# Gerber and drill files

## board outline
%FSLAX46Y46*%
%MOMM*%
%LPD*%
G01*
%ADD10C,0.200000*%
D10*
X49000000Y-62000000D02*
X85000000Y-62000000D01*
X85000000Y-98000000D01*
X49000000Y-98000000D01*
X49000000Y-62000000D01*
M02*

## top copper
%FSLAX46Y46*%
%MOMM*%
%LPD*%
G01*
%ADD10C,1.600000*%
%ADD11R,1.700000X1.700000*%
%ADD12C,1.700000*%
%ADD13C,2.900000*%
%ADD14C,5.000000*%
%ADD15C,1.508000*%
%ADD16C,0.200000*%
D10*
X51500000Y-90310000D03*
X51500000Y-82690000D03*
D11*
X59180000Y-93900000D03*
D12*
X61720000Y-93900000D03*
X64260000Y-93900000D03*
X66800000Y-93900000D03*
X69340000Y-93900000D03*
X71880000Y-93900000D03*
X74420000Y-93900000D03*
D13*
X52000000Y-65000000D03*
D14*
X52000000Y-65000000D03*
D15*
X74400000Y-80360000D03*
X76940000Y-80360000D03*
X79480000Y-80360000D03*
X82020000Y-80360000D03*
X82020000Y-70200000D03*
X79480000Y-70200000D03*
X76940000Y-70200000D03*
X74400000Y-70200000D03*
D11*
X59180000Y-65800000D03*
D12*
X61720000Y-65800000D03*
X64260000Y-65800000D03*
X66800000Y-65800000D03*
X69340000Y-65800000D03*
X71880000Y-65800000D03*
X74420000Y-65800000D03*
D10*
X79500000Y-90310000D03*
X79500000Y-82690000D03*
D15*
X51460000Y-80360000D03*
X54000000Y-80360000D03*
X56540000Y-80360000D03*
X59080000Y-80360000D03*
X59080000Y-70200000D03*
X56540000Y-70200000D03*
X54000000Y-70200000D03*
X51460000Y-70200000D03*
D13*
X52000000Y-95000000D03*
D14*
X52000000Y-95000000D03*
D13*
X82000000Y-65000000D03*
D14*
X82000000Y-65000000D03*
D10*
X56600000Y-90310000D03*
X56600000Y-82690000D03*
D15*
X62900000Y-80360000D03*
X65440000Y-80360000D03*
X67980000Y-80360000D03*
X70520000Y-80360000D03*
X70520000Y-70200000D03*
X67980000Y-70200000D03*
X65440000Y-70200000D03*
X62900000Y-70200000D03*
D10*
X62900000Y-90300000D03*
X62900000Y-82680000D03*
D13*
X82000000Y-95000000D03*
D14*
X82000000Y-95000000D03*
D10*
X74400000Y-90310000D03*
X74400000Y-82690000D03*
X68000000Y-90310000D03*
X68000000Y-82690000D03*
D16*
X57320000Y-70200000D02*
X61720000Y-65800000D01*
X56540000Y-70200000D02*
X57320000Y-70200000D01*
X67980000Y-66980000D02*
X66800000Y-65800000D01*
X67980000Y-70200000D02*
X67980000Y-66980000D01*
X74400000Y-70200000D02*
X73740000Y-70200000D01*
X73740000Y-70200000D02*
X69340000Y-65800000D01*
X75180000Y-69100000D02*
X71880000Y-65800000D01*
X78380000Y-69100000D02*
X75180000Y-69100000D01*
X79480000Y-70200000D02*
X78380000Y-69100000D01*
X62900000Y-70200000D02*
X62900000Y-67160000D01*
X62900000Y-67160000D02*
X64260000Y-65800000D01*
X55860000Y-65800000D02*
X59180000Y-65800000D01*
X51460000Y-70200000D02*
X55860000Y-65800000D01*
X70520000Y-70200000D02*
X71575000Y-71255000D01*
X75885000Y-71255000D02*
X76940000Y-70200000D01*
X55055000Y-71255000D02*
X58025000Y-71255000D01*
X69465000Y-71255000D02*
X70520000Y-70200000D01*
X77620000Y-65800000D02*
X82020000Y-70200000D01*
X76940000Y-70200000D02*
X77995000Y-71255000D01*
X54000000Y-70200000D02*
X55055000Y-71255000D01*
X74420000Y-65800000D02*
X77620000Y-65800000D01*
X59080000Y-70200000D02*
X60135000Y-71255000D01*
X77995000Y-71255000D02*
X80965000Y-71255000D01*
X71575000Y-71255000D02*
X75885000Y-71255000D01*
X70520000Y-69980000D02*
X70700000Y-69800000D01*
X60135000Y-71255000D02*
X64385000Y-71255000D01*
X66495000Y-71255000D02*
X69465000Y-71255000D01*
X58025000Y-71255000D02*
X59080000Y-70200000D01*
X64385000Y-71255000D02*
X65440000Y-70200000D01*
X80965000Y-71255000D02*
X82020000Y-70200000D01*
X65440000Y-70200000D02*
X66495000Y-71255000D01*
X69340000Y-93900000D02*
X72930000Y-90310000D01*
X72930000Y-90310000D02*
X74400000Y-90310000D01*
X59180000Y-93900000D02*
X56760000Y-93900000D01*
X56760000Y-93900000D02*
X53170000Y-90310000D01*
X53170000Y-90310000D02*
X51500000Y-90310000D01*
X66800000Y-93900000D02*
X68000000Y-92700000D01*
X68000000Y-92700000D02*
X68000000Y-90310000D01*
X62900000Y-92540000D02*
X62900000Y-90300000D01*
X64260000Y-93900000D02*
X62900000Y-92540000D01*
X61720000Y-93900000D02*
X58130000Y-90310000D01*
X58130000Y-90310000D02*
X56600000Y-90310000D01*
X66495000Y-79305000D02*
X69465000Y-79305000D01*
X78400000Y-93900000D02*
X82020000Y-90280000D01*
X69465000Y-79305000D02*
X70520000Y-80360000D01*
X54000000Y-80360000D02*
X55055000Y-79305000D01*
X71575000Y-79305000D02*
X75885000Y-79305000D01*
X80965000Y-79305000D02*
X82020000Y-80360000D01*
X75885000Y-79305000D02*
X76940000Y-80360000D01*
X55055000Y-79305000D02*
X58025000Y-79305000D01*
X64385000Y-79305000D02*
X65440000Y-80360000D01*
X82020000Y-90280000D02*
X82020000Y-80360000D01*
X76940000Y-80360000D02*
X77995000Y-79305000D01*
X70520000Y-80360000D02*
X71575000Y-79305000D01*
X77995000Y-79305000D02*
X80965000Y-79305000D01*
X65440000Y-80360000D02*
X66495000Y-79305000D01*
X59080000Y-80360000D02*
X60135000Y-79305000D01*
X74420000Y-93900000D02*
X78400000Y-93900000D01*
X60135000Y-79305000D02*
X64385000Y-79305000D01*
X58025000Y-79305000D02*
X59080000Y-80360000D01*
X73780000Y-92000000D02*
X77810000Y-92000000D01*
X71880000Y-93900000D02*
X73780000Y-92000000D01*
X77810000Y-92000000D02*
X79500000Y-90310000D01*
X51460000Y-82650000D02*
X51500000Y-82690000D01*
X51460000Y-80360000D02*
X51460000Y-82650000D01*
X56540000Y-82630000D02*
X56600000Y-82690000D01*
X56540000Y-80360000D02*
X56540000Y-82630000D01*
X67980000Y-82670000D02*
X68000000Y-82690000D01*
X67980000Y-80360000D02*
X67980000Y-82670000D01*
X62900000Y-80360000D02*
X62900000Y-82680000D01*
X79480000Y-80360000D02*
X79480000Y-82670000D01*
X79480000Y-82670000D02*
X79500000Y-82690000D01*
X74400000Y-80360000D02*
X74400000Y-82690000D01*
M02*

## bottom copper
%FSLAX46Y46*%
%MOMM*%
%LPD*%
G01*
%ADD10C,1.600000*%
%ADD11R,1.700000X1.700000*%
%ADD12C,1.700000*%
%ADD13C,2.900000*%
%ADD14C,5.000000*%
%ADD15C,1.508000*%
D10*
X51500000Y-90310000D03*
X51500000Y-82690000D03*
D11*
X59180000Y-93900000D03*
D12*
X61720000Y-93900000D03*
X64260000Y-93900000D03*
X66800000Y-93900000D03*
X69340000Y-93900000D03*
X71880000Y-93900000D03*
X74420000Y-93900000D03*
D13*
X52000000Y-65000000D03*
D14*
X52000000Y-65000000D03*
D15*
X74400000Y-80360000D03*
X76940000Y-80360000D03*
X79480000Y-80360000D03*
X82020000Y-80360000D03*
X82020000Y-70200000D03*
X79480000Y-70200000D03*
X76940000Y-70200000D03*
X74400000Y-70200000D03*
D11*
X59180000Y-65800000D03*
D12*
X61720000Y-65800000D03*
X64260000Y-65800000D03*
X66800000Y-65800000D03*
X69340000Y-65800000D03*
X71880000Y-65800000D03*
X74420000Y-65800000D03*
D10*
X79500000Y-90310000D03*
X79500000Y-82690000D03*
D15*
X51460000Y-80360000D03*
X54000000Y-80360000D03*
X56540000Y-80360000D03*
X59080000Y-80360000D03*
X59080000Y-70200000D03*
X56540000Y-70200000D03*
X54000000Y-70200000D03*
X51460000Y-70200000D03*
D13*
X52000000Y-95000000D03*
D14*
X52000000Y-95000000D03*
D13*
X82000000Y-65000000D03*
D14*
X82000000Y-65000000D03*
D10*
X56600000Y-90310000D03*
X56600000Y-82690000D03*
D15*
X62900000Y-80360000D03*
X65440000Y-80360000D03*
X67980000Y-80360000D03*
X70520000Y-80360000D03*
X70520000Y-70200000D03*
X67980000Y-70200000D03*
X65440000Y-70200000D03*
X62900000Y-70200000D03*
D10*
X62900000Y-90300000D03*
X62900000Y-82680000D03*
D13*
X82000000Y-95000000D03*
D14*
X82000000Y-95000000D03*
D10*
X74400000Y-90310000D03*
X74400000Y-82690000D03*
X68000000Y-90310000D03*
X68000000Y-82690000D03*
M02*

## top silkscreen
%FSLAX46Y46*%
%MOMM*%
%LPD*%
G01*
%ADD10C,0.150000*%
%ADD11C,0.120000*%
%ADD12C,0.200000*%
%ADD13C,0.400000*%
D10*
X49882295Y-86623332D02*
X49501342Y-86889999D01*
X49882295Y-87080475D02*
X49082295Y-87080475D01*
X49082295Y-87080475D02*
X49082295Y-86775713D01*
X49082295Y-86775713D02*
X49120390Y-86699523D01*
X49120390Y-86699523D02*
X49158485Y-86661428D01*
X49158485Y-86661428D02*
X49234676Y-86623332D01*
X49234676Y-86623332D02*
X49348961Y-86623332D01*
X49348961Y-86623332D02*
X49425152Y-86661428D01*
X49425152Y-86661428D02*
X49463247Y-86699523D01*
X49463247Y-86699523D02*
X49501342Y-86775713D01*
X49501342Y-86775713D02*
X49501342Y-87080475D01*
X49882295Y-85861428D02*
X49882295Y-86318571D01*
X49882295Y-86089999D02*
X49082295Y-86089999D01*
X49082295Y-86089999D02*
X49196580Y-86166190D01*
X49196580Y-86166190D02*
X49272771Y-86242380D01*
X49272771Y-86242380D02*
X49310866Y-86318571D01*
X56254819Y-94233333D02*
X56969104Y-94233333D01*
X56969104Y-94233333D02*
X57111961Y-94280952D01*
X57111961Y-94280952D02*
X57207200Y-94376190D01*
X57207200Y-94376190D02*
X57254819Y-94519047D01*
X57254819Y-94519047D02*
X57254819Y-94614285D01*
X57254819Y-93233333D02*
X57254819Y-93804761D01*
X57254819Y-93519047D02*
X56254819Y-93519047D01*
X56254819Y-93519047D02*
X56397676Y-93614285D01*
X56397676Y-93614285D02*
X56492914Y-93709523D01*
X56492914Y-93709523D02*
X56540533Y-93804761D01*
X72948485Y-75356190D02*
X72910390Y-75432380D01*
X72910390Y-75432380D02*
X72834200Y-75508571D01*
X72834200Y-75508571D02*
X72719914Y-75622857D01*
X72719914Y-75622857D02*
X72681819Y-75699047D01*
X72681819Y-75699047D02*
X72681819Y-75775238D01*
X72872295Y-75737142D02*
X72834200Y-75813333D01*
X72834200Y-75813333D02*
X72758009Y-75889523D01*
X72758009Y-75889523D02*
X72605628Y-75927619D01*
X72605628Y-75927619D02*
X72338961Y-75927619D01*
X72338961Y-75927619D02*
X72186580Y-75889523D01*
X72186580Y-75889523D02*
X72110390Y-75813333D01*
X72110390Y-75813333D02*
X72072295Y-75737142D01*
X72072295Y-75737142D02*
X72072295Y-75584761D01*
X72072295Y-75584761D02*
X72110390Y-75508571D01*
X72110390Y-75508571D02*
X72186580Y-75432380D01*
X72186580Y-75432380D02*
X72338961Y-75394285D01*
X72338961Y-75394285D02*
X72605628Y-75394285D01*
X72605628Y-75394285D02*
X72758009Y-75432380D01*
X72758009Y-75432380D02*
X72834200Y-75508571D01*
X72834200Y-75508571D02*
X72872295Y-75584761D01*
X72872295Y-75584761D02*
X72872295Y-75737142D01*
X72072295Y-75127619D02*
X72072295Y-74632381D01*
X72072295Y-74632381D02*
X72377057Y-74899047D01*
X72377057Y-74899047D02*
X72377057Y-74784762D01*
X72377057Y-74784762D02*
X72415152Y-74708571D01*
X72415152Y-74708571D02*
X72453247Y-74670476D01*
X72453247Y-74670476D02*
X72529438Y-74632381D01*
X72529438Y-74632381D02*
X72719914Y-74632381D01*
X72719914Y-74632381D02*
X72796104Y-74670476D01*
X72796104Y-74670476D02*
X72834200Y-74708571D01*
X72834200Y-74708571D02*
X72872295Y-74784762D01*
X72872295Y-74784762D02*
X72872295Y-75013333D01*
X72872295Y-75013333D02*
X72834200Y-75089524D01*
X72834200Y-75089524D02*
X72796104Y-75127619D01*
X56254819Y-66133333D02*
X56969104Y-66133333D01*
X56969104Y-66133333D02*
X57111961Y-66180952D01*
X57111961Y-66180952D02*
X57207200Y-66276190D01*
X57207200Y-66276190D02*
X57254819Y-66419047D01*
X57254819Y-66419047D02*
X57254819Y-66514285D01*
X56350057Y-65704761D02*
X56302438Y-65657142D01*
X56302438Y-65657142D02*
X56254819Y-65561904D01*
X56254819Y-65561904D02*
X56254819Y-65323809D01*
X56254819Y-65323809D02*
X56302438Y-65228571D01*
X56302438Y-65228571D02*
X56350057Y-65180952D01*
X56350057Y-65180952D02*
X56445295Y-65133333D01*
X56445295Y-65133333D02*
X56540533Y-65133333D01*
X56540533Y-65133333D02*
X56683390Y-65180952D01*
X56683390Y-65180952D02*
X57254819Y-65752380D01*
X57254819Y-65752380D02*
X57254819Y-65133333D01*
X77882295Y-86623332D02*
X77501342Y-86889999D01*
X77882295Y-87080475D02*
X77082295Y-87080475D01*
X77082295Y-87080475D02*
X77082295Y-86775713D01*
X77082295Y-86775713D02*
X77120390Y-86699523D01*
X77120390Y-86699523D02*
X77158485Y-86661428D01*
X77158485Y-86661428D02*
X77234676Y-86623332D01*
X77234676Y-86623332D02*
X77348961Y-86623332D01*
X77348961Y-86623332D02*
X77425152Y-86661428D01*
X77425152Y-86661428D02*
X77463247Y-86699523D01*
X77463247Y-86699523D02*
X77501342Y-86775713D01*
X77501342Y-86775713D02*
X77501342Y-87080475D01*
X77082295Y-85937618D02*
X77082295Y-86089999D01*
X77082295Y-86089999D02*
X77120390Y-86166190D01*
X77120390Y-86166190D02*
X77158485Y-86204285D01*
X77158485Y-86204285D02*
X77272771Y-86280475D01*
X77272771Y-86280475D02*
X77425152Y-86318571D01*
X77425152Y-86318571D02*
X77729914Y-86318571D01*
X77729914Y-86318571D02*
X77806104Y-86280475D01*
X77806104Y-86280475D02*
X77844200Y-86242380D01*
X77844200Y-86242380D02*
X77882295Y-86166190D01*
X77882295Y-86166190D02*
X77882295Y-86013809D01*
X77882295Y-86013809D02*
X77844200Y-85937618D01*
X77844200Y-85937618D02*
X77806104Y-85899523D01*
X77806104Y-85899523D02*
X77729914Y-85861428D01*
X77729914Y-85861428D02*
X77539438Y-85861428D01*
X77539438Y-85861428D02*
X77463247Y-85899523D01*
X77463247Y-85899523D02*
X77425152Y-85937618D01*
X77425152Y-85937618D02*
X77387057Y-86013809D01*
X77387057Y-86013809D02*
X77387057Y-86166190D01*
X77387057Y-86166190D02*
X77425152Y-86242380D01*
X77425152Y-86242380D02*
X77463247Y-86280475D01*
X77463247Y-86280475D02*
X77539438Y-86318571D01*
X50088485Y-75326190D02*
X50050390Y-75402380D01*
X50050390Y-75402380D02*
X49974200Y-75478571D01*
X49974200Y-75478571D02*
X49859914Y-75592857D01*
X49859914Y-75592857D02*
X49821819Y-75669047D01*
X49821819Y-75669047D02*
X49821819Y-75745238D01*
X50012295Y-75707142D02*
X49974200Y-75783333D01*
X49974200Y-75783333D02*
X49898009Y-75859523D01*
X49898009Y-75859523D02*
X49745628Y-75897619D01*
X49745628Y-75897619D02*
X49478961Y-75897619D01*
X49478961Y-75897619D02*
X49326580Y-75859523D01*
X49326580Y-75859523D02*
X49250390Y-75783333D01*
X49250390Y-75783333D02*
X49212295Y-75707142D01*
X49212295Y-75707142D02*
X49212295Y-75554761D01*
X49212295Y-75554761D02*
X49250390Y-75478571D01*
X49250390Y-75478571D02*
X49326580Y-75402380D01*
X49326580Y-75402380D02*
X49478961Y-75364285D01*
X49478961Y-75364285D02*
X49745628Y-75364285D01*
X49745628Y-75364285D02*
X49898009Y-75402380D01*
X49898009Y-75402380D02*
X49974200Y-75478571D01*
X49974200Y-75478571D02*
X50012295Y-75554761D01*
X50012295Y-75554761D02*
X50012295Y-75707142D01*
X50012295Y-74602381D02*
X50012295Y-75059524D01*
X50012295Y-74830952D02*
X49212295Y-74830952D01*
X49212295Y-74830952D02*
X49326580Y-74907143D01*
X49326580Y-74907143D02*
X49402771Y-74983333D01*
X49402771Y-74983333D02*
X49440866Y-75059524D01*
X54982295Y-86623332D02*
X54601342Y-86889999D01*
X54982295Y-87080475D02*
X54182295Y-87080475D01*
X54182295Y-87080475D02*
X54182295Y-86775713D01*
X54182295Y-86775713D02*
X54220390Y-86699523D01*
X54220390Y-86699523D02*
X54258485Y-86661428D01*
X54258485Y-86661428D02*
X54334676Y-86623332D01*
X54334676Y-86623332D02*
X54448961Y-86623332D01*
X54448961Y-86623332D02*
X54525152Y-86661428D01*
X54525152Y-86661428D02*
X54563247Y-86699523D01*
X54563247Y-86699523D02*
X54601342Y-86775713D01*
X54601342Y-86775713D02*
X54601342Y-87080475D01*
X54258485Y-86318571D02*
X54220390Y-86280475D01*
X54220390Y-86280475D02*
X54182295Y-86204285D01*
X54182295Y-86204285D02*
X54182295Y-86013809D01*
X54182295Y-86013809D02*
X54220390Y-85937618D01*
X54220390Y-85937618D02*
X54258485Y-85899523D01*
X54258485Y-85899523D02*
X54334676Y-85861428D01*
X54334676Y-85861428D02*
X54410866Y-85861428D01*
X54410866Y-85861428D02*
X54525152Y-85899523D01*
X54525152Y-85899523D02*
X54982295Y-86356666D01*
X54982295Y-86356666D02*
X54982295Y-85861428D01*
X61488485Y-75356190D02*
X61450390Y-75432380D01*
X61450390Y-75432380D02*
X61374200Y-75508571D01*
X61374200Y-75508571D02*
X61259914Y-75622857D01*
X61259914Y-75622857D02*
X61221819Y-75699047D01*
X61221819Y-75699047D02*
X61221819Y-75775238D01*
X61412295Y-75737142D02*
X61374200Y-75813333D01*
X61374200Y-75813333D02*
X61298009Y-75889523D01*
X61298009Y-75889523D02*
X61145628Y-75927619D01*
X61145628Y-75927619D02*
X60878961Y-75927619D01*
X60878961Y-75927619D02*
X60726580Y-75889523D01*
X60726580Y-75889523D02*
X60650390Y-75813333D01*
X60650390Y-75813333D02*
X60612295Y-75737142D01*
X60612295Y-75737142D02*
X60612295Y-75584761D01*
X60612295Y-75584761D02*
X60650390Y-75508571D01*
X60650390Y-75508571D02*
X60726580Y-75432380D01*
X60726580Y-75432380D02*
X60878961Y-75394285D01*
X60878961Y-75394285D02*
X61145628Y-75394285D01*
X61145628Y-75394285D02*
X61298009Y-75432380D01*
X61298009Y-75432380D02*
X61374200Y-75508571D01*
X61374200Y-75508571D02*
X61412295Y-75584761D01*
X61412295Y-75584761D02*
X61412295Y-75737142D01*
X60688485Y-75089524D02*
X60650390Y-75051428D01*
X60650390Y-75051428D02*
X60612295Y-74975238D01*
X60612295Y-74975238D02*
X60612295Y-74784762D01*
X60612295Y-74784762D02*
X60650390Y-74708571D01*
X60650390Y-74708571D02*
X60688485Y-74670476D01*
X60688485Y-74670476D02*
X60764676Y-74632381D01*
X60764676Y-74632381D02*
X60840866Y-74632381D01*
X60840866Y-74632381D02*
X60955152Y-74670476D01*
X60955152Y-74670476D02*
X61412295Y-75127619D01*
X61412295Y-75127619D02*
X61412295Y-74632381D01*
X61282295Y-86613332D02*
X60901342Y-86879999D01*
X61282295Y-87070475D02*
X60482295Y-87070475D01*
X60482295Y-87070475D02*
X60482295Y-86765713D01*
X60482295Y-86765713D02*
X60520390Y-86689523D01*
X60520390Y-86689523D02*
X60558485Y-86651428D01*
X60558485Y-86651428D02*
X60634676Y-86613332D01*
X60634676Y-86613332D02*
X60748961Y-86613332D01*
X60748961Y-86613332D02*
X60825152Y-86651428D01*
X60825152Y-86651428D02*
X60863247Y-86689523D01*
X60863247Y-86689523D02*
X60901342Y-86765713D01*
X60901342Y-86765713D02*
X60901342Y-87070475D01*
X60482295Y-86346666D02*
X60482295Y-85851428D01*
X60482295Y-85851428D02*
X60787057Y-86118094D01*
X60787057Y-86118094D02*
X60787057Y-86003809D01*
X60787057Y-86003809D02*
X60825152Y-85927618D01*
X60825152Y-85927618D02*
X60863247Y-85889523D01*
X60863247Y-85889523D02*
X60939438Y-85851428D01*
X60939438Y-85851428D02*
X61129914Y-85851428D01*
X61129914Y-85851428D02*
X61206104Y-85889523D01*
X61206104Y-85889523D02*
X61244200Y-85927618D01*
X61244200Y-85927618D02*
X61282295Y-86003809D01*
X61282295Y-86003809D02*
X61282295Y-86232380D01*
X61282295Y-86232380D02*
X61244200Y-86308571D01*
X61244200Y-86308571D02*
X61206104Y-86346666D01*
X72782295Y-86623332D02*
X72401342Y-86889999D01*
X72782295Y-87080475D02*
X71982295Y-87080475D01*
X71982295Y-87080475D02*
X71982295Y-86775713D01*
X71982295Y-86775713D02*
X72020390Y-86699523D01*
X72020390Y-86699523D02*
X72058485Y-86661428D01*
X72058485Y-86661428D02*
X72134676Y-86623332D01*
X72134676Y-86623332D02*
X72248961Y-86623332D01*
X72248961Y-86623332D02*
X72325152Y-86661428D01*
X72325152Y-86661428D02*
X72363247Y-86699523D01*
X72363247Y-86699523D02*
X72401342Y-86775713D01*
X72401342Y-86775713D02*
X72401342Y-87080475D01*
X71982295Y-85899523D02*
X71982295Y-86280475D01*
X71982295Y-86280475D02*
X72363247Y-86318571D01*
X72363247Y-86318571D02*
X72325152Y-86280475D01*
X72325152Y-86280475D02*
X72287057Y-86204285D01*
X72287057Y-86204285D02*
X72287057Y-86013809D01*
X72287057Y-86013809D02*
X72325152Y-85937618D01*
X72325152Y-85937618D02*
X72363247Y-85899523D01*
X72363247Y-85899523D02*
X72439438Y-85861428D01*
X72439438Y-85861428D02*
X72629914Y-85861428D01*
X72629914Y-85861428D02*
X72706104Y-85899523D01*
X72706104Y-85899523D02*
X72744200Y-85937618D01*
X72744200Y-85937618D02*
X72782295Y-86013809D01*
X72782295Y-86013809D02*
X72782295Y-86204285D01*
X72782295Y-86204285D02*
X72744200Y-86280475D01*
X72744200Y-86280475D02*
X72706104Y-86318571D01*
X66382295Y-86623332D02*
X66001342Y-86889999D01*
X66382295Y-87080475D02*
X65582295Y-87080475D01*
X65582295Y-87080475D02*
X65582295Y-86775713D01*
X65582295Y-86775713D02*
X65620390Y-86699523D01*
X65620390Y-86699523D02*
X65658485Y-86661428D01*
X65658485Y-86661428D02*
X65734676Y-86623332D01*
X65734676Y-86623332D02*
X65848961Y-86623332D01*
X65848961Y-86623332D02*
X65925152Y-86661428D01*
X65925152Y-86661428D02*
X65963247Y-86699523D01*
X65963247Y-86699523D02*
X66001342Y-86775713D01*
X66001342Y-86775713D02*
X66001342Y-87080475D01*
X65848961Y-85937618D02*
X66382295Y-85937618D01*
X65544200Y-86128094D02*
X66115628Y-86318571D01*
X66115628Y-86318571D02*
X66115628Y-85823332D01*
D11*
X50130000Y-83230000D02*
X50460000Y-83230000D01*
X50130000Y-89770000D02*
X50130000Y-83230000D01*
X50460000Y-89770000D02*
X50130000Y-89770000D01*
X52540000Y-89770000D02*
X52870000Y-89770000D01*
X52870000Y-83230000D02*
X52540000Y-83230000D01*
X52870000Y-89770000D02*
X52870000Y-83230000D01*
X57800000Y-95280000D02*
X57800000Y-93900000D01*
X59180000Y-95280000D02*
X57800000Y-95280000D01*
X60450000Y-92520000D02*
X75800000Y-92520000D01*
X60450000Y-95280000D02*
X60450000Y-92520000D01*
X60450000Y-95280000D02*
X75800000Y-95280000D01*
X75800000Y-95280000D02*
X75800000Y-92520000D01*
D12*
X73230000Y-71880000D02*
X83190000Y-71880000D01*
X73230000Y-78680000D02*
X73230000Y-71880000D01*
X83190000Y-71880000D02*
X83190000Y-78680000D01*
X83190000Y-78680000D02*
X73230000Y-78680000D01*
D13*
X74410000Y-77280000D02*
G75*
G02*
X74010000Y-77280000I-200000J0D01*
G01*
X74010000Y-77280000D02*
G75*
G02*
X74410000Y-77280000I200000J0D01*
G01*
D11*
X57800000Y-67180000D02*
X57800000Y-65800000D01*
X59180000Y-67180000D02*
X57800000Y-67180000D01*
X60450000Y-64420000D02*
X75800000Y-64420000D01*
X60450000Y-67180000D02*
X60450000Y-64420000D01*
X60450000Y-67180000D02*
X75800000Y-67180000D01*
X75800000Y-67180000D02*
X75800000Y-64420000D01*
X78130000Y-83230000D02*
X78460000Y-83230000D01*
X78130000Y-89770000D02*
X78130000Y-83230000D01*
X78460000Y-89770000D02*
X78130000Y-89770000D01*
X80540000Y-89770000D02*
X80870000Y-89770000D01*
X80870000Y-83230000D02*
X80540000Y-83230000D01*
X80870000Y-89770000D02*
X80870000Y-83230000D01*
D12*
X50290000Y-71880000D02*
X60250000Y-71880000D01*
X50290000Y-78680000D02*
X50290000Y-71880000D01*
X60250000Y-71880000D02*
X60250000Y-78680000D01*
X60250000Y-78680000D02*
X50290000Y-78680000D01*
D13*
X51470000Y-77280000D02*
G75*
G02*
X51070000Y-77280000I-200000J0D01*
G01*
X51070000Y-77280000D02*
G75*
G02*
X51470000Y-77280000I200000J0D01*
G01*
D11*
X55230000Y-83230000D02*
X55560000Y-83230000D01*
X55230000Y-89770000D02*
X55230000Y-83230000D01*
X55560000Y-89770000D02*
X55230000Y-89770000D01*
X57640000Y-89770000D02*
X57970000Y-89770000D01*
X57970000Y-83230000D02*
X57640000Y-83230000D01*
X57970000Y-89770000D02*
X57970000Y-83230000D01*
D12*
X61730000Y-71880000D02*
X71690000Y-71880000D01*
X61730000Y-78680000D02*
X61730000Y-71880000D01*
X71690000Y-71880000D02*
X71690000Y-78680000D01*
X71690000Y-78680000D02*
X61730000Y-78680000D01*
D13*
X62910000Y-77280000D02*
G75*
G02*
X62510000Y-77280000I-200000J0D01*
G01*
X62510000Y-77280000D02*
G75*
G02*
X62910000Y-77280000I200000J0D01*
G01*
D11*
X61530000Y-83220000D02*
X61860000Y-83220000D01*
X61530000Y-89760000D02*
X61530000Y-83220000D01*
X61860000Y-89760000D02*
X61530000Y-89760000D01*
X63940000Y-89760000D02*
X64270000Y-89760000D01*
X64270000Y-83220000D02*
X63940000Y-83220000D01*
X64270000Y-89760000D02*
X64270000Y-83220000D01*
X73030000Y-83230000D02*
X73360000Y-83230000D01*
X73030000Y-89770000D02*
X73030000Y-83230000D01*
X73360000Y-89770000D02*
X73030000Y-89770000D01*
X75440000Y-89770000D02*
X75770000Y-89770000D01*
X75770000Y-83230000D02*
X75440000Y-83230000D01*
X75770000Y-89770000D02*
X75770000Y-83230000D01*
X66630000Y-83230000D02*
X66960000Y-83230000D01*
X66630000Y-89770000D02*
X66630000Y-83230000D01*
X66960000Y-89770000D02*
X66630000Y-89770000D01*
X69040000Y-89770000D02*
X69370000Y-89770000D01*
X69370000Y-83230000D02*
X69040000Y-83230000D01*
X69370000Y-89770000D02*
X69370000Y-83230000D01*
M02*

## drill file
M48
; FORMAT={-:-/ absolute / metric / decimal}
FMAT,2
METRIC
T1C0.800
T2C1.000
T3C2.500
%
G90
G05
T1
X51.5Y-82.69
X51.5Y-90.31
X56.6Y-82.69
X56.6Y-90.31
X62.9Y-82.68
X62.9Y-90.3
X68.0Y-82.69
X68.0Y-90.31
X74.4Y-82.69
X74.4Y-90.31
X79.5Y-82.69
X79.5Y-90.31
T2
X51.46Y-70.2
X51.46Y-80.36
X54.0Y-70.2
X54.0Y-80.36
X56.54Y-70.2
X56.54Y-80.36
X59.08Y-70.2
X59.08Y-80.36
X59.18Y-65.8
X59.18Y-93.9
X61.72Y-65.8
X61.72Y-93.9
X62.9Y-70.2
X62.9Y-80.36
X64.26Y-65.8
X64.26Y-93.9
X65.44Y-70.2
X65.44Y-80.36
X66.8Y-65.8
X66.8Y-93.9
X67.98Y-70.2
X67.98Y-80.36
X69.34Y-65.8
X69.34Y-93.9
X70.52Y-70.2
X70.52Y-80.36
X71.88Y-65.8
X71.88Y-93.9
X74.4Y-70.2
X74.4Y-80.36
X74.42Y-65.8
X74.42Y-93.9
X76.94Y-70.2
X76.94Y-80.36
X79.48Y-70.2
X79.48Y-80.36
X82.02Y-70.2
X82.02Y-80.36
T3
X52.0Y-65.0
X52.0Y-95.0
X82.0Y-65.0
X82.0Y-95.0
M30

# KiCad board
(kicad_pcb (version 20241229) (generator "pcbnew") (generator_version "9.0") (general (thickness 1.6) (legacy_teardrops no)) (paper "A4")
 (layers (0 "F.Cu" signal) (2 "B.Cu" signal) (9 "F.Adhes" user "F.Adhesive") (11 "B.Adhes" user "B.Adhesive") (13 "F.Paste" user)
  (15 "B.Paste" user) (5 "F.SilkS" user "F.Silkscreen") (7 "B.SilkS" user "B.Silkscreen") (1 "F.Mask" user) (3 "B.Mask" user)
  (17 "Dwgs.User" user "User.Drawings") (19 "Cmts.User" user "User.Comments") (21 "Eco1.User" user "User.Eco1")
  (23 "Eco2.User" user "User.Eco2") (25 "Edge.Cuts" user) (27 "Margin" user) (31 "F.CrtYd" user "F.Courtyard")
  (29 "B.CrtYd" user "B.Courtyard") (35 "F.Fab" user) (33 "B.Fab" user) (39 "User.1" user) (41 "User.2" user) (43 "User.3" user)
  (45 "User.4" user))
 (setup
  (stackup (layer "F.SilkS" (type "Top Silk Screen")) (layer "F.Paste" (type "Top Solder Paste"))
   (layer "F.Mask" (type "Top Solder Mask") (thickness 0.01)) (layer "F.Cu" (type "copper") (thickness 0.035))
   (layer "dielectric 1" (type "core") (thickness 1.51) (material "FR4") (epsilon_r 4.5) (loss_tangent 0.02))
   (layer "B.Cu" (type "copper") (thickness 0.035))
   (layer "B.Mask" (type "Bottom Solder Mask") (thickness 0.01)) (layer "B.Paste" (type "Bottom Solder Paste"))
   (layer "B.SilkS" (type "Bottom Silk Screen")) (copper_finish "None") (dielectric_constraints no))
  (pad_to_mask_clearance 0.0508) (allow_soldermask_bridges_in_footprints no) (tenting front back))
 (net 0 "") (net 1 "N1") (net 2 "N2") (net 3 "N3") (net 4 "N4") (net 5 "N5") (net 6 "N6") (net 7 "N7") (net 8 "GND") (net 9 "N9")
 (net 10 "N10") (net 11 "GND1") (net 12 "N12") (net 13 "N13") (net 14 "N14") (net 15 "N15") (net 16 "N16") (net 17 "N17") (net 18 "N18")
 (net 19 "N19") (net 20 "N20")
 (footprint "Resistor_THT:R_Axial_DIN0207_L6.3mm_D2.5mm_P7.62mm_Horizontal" (layer "F.Cu") (at 51.5 90.31 90)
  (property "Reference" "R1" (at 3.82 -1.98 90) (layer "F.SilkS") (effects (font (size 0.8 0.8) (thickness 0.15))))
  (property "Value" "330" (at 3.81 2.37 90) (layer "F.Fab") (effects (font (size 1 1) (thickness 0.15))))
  (fp_line (start 7.08 -1.37) (end 7.08 -1.04) (stroke (width 0.12) (type solid)) (layer "F.SilkS"))
  (fp_line (start 0.54 -1.37) (end 7.08 -1.37) (stroke (width 0.12) (type solid)) (layer "F.SilkS"))
  (fp_line (start 0.54 -1.04) (end 0.54 -1.37) (stroke (width 0.12) (type solid)) (layer "F.SilkS"))
  (fp_line (start 0.54 1.04) (end 0.54 1.37) (stroke (width 0.12) (type solid)) (layer "F.SilkS"))
  (fp_line (start 7.08 1.37) (end 7.08 1.04) (stroke (width 0.12) (type solid)) (layer "F.SilkS"))
  (fp_line (start 0.54 1.37) (end 7.08 1.37) (stroke (width 0.12) (type solid)) (layer "F.SilkS"))
  (pad "1" thru_hole circle (at 0 0 90) (size 1.6 1.6) (drill 0.8) (layers "*.Cu" "*.Mask") (remove_unused_layers no) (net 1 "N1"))
  (pad "2" thru_hole circle (at 7.62 0 90) (size 1.6 1.6) (drill 0.8) (layers "*.Cu" "*.Mask") (remove_unused_layers no) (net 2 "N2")))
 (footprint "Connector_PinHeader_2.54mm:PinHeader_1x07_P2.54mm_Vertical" (layer "F.Cu") (at 59.18 93.9 90)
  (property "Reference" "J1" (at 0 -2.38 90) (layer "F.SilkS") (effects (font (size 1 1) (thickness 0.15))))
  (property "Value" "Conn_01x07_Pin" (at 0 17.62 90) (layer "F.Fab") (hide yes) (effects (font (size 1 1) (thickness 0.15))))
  (fp_line (start -1.38 -1.38) (end 0 -1.38) (stroke (width 0.12) (type solid)) (layer "F.SilkS"))
  (fp_line (start -1.38 0) (end -1.38 -1.38) (stroke (width 0.12) (type solid)) (layer "F.SilkS"))
  (fp_line (start 1.38 1.27) (end 1.38 16.62) (stroke (width 0.12) (type solid)) (layer "F.SilkS"))
  (fp_line (start -1.38 1.27) (end 1.38 1.27) (stroke (width 0.12) (type solid)) (layer "F.SilkS"))
  (fp_line (start -1.38 1.27) (end -1.38 16.62) (stroke (width 0.12) (type solid)) (layer "F.SilkS"))
  (fp_line (start -1.38 16.62) (end 1.38 16.62) (stroke (width 0.12) (type solid)) (layer "F.SilkS"))
  (pad "1" thru_hole rect (at 0 0 90) (size 1.7 1.7) (drill 1) (layers "*.Cu" "*.Mask") (remove_unused_layers no) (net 1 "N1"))
  (pad "2" thru_hole circle (at 0 2.54 90) (size 1.7 1.7) (drill 1) (layers "*.Cu" "*.Mask") (remove_unused_layers no) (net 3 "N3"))
  (pad "3" thru_hole circle (at 0 5.08 90) (size 1.7 1.7) (drill 1) (layers "*.Cu" "*.Mask") (remove_unused_layers no) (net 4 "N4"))
  (pad "4" thru_hole circle (at 0 7.62 90) (size 1.7 1.7) (drill 1) (layers "*.Cu" "*.Mask") (remove_unused_layers no) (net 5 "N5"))
  (pad "5" thru_hole circle (at 0 10.16 90) (size 1.7 1.7) (drill 1) (layers "*.Cu" "*.Mask") (remove_unused_layers no) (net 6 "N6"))
  (pad "6" thru_hole circle (at 0 12.7 90) (size 1.7 1.7) (drill 1) (layers "*.Cu" "*.Mask") (remove_unused_layers no) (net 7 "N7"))
  (pad "7" thru_hole circle (at 0 15.24 90) (size 1.7 1.7) (drill 1) (layers "*.Cu" "*.Mask") (remove_unused_layers no) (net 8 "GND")))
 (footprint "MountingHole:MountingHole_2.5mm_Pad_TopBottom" (layer "F.Cu") (at 52 65)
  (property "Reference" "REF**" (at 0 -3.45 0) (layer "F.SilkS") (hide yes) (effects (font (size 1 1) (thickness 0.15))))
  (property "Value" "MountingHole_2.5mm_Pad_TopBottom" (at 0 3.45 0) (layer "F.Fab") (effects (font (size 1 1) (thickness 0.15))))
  (pad "1" thru_hole circle (at 0 0) (size 2.9 2.9) (drill 2.5) (layers "*.Cu" "*.Mask") (remove_unused_layers no) (zone_connect 2))
  (pad "1" connect circle (at 0 0) (size 5 5) (layers "F.Cu" "F.Mask") (zone_connect 2))
  (pad "1" connect circle (at 0 0) (size 5 5) (layers "B.Cu" "B.Mask") (zone_connect 2)))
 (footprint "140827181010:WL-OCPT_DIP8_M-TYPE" (layer "F.Cu") (at 78.21 75.28)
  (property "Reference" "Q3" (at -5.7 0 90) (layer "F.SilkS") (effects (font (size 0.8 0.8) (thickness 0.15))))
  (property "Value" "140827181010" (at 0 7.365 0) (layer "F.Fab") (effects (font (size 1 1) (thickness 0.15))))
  (fp_line (start -4.98 -3.4) (end 4.98 -3.4) (stroke (width 0.2) (type solid)) (layer "F.SilkS"))
  (fp_line (start -4.98 3.4) (end -4.98 -3.4) (stroke (width 0.2) (type solid)) (layer "F.SilkS"))
  (fp_line (start 4.98 -3.4) (end 4.98 3.4) (stroke (width 0.2) (type solid)) (layer "F.SilkS"))
  (fp_line (start 4.98 3.4) (end -4.98 3.4) (stroke (width 0.2) (type solid)) (layer "F.SilkS"))
  (fp_circle (center -4 2) (end -3.8 2) (stroke (width 0.4) (type solid)) (fill no) (layer "F.SilkS"))
  (pad "1" thru_hole circle (at -3.81 5.08) (size 1.508 1.508) (drill 1) (layers "*.Cu" "*.Mask") (remove_unused_layers no) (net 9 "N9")
   (solder_mask_margin 0.102))
  (pad "2" thru_hole circle (at -1.27 5.08) (size 1.508 1.508) (drill 1) (layers "*.Cu" "*.Mask") (remove_unused_layers no) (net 8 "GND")
   (solder_mask_margin 0.102))
  (pad "3" thru_hole circle (at 1.27 5.08) (size 1.508 1.508) (drill 1) (layers "*.Cu" "*.Mask") (remove_unused_layers no) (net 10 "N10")
   (solder_mask_margin 0.102))
  (pad "4" thru_hole circle (at 3.81 5.08) (size 1.508 1.508) (drill 1) (layers "*.Cu" "*.Mask") (remove_unused_layers no) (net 8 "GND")
   (solder_mask_margin 0.102))
  (pad "5" thru_hole circle (at 3.81 -5.08) (size 1.508 1.508) (drill 1) (layers "*.Cu" "*.Mask") (remove_unused_layers no) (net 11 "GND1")
   (solder_mask_margin 0.102))
  (pad "6" thru_hole circle (at 1.27 -5.08) (size 1.508 1.508) (drill 1) (layers "*.Cu" "*.Mask") (remove_unused_layers no) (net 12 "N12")
   (solder_mask_margin 0.102))
  (pad "7" thru_hole circle (at -1.27 -5.08) (size 1.508 1.508) (drill 1) (layers "*.Cu" "*.Mask") (remove_unused_layers no) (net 11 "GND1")
   (solder_mask_margin 0.102))
  (pad "8" thru_hole circle (at -3.81 -5.08) (size 1.508 1.508) (drill 1) (layers "*.Cu" "*.Mask") (remove_unused_layers no) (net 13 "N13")
   (solder_mask_margin 0.102)))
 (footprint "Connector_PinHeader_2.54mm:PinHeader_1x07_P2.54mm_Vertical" (layer "F.Cu") (at 59.18 65.8 90)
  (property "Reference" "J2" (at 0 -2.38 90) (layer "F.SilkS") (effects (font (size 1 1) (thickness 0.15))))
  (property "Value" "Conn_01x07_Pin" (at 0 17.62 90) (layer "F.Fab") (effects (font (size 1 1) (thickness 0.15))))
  (fp_line (start -1.38 -1.38) (end 0 -1.38) (stroke (width 0.12) (type solid)) (layer "F.SilkS"))
  (fp_line (start -1.38 0) (end -1.38 -1.38) (stroke (width 0.12) (type solid)) (layer "F.SilkS"))
  (fp_line (start 1.38 1.27) (end 1.38 16.62) (stroke (width 0.12) (type solid)) (layer "F.SilkS"))
  (fp_line (start -1.38 1.27) (end 1.38 1.27) (stroke (width 0.12) (type solid)) (layer "F.SilkS"))
  (fp_line (start -1.38 1.27) (end -1.38 16.62) (stroke (width 0.12) (type solid)) (layer "F.SilkS"))
  (fp_line (start -1.38 16.62) (end 1.38 16.62) (stroke (width 0.12) (type solid)) (layer "F.SilkS"))
  (pad "1" thru_hole rect (at 0 0 90) (size 1.7 1.7) (drill 1) (layers "*.Cu" "*.Mask") (remove_unused_layers no) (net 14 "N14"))
  (pad "2" thru_hole circle (at 0 2.54 90) (size 1.7 1.7) (drill 1) (layers "*.Cu" "*.Mask") (remove_unused_layers no) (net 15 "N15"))
  (pad "3" thru_hole circle (at 0 5.08 90) (size 1.7 1.7) (drill 1) (layers "*.Cu" "*.Mask") (remove_unused_layers no) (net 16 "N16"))
  (pad "4" thru_hole circle (at 0 7.62 90) (size 1.7 1.7) (drill 1) (layers "*.Cu" "*.Mask") (remove_unused_layers no) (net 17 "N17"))
  (pad "5" thru_hole circle (at 0 10.16 90) (size 1.7 1.7) (drill 1) (layers "*.Cu" "*.Mask") (remove_unused_layers no) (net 13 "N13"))
  (pad "6" thru_hole circle (at 0 12.7 90) (size 1.7 1.7) (drill 1) (layers "*.Cu" "*.Mask") (remove_unused_layers no) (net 12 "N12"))
  (pad "7" thru_hole circle (at 0 15.24 90) (size 1.7 1.7) (drill 1) (layers "*.Cu" "*.Mask") (remove_unused_layers no) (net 11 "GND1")))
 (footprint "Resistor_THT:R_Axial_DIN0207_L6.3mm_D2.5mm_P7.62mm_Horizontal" (layer "F.Cu") (at 79.5 90.31 90)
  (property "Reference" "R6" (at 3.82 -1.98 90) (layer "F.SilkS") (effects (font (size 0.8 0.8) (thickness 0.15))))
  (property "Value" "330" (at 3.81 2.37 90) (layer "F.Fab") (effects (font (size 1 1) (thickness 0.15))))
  (fp_line (start 7.08 -1.37) (end 7.08 -1.04) (stroke (width 0.12) (type solid)) (layer "F.SilkS"))
  (fp_line (start 0.54 -1.37) (end 7.08 -1.37) (stroke (width 0.12) (type solid)) (layer "F.SilkS"))
  (fp_line (start 0.54 -1.04) (end 0.54 -1.37) (stroke (width 0.12) (type solid)) (layer "F.SilkS"))
  (fp_line (start 0.54 1.04) (end 0.54 1.37) (stroke (width 0.12) (type solid)) (layer "F.SilkS"))
  (fp_line (start 7.08 1.37) (end 7.08 1.04) (stroke (width 0.12) (type solid)) (layer "F.SilkS"))
  (fp_line (start 0.54 1.37) (end 7.08 1.37) (stroke (width 0.12) (type solid)) (layer "F.SilkS"))
  (pad "1" thru_hole circle (at 0 0 90) (size 1.6 1.6) (drill 0.8) (layers "*.Cu" "*.Mask") (remove_unused_layers no) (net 7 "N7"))
  (pad "2" thru_hole circle (at 7.62 0 90) (size 1.6 1.6) (drill 0.8) (layers "*.Cu" "*.Mask") (remove_unused_layers no) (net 10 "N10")))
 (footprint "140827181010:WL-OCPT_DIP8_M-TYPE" (layer "F.Cu") (at 55.27 75.28)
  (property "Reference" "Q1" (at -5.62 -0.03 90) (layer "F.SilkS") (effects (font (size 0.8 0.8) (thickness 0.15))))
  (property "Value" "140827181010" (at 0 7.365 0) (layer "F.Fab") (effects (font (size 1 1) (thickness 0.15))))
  (fp_line (start -4.98 -3.4) (end 4.98 -3.4) (stroke (width 0.2) (type solid)) (layer "F.SilkS"))
  (fp_line (start -4.98 3.4) (end -4.98 -3.4) (stroke (width 0.2) (type solid)) (layer "F.SilkS"))
  (fp_line (start 4.98 -3.4) (end 4.98 3.4) (stroke (width 0.2) (type solid)) (layer "F.SilkS"))
  (fp_line (start 4.98 3.4) (end -4.98 3.4) (stroke (width 0.2) (type solid)) (layer "F.SilkS"))
  (fp_circle (center -4 2) (end -3.8 2) (stroke (width 0.4) (type solid)) (fill no) (layer "F.SilkS"))
  (pad "1" thru_hole circle (at -3.81 5.08) (size 1.508 1.508) (drill 1) (layers "*.Cu" "*.Mask") (remove_unused_layers no) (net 2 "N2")
   (solder_mask_margin 0.102))
  (pad "2" thru_hole circle (at -1.27 5.08) (size 1.508 1.508) (drill 1) (layers "*.Cu" "*.Mask") (remove_unused_layers no) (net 8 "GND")
   (solder_mask_margin 0.102))
  (pad "3" thru_hole circle (at 1.27 5.08) (size 1.508 1.508) (drill 1) (layers "*.Cu" "*.Mask") (remove_unused_layers no) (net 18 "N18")
   (solder_mask_margin 0.102))
  (pad "4" thru_hole circle (at 3.81 5.08) (size 1.508 1.508) (drill 1) (layers "*.Cu" "*.Mask") (remove_unused_layers no) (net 8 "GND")
   (solder_mask_margin 0.102))
  (pad "5" thru_hole circle (at 3.81 -5.08) (size 1.508 1.508) (drill 1) (layers "*.Cu" "*.Mask") (remove_unused_layers no) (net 11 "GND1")
   (solder_mask_margin 0.102))
  (pad "6" thru_hole circle (at 1.27 -5.08) (size 1.508 1.508) (drill 1) (layers "*.Cu" "*.Mask") (remove_unused_layers no) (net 15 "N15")
   (solder_mask_margin 0.102))
  (pad "7" thru_hole circle (at -1.27 -5.08) (size 1.508 1.508) (drill 1) (layers "*.Cu" "*.Mask") (remove_unused_layers no) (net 11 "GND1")
   (solder_mask_margin 0.102))
  (pad "8" thru_hole circle (at -3.81 -5.08) (size 1.508 1.508) (drill 1) (layers "*.Cu" "*.Mask") (remove_unused_layers no) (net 14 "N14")
   (solder_mask_margin 0.102)))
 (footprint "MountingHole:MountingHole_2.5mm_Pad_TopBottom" (layer "F.Cu") (at 52 95)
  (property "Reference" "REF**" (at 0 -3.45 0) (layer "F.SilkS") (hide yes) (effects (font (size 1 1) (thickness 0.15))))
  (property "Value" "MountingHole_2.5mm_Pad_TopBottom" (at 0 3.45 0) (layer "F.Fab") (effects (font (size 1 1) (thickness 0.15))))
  (pad "1" thru_hole circle (at 0 0) (size 2.9 2.9) (drill 2.5) (layers "*.Cu" "*.Mask") (remove_unused_layers no) (zone_connect 2))
  (pad "1" connect circle (at 0 0) (size 5 5) (layers "F.Cu" "F.Mask") (zone_connect 2))
  (pad "1" connect circle (at 0 0) (size 5 5) (layers "B.Cu" "B.Mask") (zone_connect 2)))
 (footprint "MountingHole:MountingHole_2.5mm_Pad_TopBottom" (layer "F.Cu") (at 82 65)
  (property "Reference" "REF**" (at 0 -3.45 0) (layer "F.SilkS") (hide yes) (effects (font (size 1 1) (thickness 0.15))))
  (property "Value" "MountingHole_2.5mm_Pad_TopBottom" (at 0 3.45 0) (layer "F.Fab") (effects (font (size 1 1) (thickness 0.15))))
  (pad "1" thru_hole circle (at 0 0) (size 2.9 2.9) (drill 2.5) (layers "*.Cu" "*.Mask") (remove_unused_layers no) (zone_connect 2))
  (pad "1" connect circle (at 0 0) (size 5 5) (layers "F.Cu" "F.Mask") (zone_connect 2))
  (pad "1" connect circle (at 0 0) (size 5 5) (layers "B.Cu" "B.Mask") (zone_connect 2)))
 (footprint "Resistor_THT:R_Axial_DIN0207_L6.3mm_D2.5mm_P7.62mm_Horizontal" (layer "F.Cu") (at 56.6 90.31 90)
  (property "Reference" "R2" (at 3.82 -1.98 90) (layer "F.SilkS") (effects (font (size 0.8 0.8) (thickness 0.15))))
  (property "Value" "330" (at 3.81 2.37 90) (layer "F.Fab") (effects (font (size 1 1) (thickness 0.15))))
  (fp_line (start 7.08 -1.37) (end 7.08 -1.04) (stroke (width 0.12) (type solid)) (layer "F.SilkS"))
  (fp_line (start 0.54 -1.37) (end 7.08 -1.37) (stroke (width 0.12) (type solid)) (layer "F.SilkS"))
  (fp_line (start 0.54 -1.04) (end 0.54 -1.37) (stroke (width 0.12) (type solid)) (layer "F.SilkS"))
  (fp_line (start 0.54 1.04) (end 0.54 1.37) (stroke (width 0.12) (type solid)) (layer "F.SilkS"))
  (fp_line (start 7.08 1.37) (end 7.08 1.04) (stroke (width 0.12) (type solid)) (layer "F.SilkS"))
  (fp_line (start 0.54 1.37) (end 7.08 1.37) (stroke (width 0.12) (type solid)) (layer "F.SilkS"))
  (pad "1" thru_hole circle (at 0 0 90) (size 1.6 1.6) (drill 0.8) (layers "*.Cu" "*.Mask") (remove_unused_layers no) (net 3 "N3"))
  (pad "2" thru_hole circle (at 7.62 0 90) (size 1.6 1.6) (drill 0.8) (layers "*.Cu" "*.Mask") (remove_unused_layers no) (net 18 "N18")))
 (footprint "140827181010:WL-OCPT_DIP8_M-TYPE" (layer "F.Cu") (at 66.71 75.28)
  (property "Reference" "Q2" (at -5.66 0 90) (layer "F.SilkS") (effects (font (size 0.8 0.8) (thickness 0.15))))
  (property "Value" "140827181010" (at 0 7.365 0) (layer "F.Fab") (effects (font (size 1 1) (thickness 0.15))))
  (fp_line (start -4.98 -3.4) (end 4.98 -3.4) (stroke (width 0.2) (type solid)) (layer "F.SilkS"))
  (fp_line (start -4.98 3.4) (end -4.98 -3.4) (stroke (width 0.2) (type solid)) (layer "F.SilkS"))
  (fp_line (start 4.98 -3.4) (end 4.98 3.4) (stroke (width 0.2) (type solid)) (layer "F.SilkS"))
  (fp_line (start 4.98 3.4) (end -4.98 3.4) (stroke (width 0.2) (type solid)) (layer "F.SilkS"))
  (fp_circle (center -4 2) (end -3.8 2) (stroke (width 0.4) (type solid)) (fill no) (layer "F.SilkS"))
  (pad "1" thru_hole circle (at -3.81 5.08) (size 1.508 1.508) (drill 1) (layers "*.Cu" "*.Mask") (remove_unused_layers no) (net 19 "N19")
   (solder_mask_margin 0.102))
  (pad "2" thru_hole circle (at -1.27 5.08) (size 1.508 1.508) (drill 1) (layers "*.Cu" "*.Mask") (remove_unused_layers no) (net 8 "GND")
   (solder_mask_margin 0.102))
  (pad "3" thru_hole circle (at 1.27 5.08) (size 1.508 1.508) (drill 1) (layers "*.Cu" "*.Mask") (remove_unused_layers no) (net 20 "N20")
   (solder_mask_margin 0.102))
  (pad "4" thru_hole circle (at 3.81 5.08) (size 1.508 1.508) (drill 1) (layers "*.Cu" "*.Mask") (remove_unused_layers no) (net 8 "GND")
   (solder_mask_margin 0.102))
  (pad "5" thru_hole circle (at 3.81 -5.08) (size 1.508 1.508) (drill 1) (layers "*.Cu" "*.Mask") (remove_unused_layers no) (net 11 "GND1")
   (solder_mask_margin 0.102))
  (pad "6" thru_hole circle (at 1.27 -5.08) (size 1.508 1.508) (drill 1) (layers "*.Cu" "*.Mask") (remove_unused_layers no) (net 17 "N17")
   (solder_mask_margin 0.102))
  (pad "7" thru_hole circle (at -1.27 -5.08) (size 1.508 1.508) (drill 1) (layers "*.Cu" "*.Mask") (remove_unused_layers no) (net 11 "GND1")
   (solder_mask_margin 0.102))
  (pad "8" thru_hole circle (at -3.81 -5.08) (size 1.508 1.508) (drill 1) (layers "*.Cu" "*.Mask") (remove_unused_layers no) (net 16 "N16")
   (solder_mask_margin 0.102)))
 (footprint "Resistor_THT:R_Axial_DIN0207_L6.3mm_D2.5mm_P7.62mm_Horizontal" (layer "F.Cu") (at 62.9 90.3 90)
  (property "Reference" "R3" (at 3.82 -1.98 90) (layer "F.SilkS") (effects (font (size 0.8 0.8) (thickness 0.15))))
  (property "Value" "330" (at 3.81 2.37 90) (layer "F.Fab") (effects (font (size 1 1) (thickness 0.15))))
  (fp_line (start 7.08 -1.37) (end 7.08 -1.04) (stroke (width 0.12) (type solid)) (layer "F.SilkS"))
  (fp_line (start 0.54 -1.37) (end 7.08 -1.37) (stroke (width 0.12) (type solid)) (layer "F.SilkS"))
  (fp_line (start 0.54 -1.04) (end 0.54 -1.37) (stroke (width 0.12) (type solid)) (layer "F.SilkS"))
  (fp_line (start 0.54 1.04) (end 0.54 1.37) (stroke (width 0.12) (type solid)) (layer "F.SilkS"))
  (fp_line (start 7.08 1.37) (end 7.08 1.04) (stroke (width 0.12) (type solid)) (layer "F.SilkS"))
  (fp_line (start 0.54 1.37) (end 7.08 1.37) (stroke (width 0.12) (type solid)) (layer "F.SilkS"))
  (pad "1" thru_hole circle (at 0 0 90) (size 1.6 1.6) (drill 0.8) (layers "*.Cu" "*.Mask") (remove_unused_layers no) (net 4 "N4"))
  (pad "2" thru_hole circle (at 7.62 0 90) (size 1.6 1.6) (drill 0.8) (layers "*.Cu" "*.Mask") (remove_unused_layers no) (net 19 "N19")))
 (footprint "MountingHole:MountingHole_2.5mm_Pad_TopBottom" (layer "F.Cu") (at 82 95)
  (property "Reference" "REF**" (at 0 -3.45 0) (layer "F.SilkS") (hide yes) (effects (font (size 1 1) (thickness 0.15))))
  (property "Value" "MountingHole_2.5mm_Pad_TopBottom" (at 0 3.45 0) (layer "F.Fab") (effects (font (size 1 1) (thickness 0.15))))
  (pad "1" thru_hole circle (at 0 0) (size 2.9 2.9) (drill 2.5) (layers "*.Cu" "*.Mask") (remove_unused_layers no) (zone_connect 2))
  (pad "1" connect circle (at 0 0) (size 5 5) (layers "F.Cu" "F.Mask") (zone_connect 2))
  (pad "1" connect circle (at 0 0) (size 5 5) (layers "B.Cu" "B.Mask") (zone_connect 2)))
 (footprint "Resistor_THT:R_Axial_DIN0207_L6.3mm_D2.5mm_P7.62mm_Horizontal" (layer "F.Cu") (at 74.4 90.31 90)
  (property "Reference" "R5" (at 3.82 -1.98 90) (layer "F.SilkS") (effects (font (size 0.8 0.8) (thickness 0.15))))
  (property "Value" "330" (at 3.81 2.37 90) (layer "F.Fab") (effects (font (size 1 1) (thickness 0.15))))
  (fp_line (start 7.08 -1.37) (end 7.08 -1.04) (stroke (width 0.12) (type solid)) (layer "F.SilkS"))
  (fp_line (start 0.54 -1.37) (end 7.08 -1.37) (stroke (width 0.12) (type solid)) (layer "F.SilkS"))
  (fp_line (start 0.54 -1.04) (end 0.54 -1.37) (stroke (width 0.12) (type solid)) (layer "F.SilkS"))
  (fp_line (start 0.54 1.04) (end 0.54 1.37) (stroke (width 0.12) (type solid)) (layer "F.SilkS"))
  (fp_line (start 7.08 1.37) (end 7.08 1.04) (stroke (width 0.12) (type solid)) (layer "F.SilkS"))
  (fp_line (start 0.54 1.37) (end 7.08 1.37) (stroke (width 0.12) (type solid)) (layer "F.SilkS"))
  (pad "1" thru_hole circle (at 0 0 90) (size 1.6 1.6) (drill 0.8) (layers "*.Cu" "*.Mask") (remove_unused_layers no) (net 6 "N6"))
  (pad "2" thru_hole circle (at 7.62 0 90) (size 1.6 1.6) (drill 0.8) (layers "*.Cu" "*.Mask") (remove_unused_layers no) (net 9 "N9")))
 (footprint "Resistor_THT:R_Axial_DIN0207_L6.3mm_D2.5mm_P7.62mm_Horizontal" (layer "F.Cu") (at 68 90.31 90)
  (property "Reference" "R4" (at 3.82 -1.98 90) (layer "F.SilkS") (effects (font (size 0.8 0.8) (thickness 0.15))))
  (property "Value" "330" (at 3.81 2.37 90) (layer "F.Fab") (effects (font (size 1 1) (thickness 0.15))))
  (fp_line (start 7.08 -1.37) (end 7.08 -1.04) (stroke (width 0.12) (type solid)) (layer "F.SilkS"))
  (fp_line (start 0.54 -1.37) (end 7.08 -1.37) (stroke (width 0.12) (type solid)) (layer "F.SilkS"))
  (fp_line (start 0.54 -1.04) (end 0.54 -1.37) (stroke (width 0.12) (type solid)) (layer "F.SilkS"))
  (fp_line (start 0.54 1.04) (end 0.54 1.37) (stroke (width 0.12) (type solid)) (layer "F.SilkS"))
  (fp_line (start 7.08 1.37) (end 7.08 1.04) (stroke (width 0.12) (type solid)) (layer "F.SilkS"))
  (fp_line (start 0.54 1.37) (end 7.08 1.37) (stroke (width 0.12) (type solid)) (layer "F.SilkS"))
  (pad "1" thru_hole circle (at 0 0 90) (size 1.6 1.6) (drill 0.8) (layers "*.Cu" "*.Mask") (remove_unused_layers no) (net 5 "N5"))
  (pad "2" thru_hole circle (at 7.62 0 90) (size 1.6 1.6) (drill 0.8) (layers "*.Cu" "*.Mask") (remove_unused_layers no) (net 20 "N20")))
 (gr_rect (start 49 62) (end 85 98) (stroke (width 0.2) (type default)) (fill no) (layer "Edge.Cuts"))
 (segment (start 57.32 70.2) (end 61.72 65.8) (width 0.2) (layer "F.Cu") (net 15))
 (segment (start 56.54 70.2) (end 57.32 70.2) (width 0.2) (layer "F.Cu") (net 15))
 (segment (start 67.98 66.98) (end 66.8 65.8) (width 0.2) (layer "F.Cu") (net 17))
 (segment (start 67.98 70.2) (end 67.98 66.98) (width 0.2) (layer "F.Cu") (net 17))
 (segment (start 74.4 70.2) (end 73.74 70.2) (width 0.2) (layer "F.Cu") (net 13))
 (segment (start 73.74 70.2) (end 69.34 65.8) (width 0.2) (layer "F.Cu") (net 13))
 (segment (start 75.18 69.1) (end 71.88 65.8) (width 0.2) (layer "F.Cu") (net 12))
 (segment (start 78.38 69.1) (end 75.18 69.1) (width 0.2) (layer "F.Cu") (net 12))
 (segment (start 79.48 70.2) (end 78.38 69.1) (width 0.2) (layer "F.Cu") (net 12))
 (segment (start 62.9 70.2) (end 62.9 67.16) (width 0.2) (layer "F.Cu") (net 16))
 (segment (start 62.9 67.16) (end 64.26 65.8) (width 0.2) (layer "F.Cu") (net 16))
 (segment (start 55.86 65.8) (end 59.18 65.8) (width 0.2) (layer "F.Cu") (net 14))
 (segment (start 51.46 70.2) (end 55.86 65.8) (width 0.2) (layer "F.Cu") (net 14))
 (segment (start 70.52 70.2) (end 71.575 71.255) (width 0.2) (layer "F.Cu") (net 11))
 (segment (start 75.885 71.255) (end 76.94 70.2) (width 0.2) (layer "F.Cu") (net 11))
 (segment (start 55.055 71.255) (end 58.025 71.255) (width 0.2) (layer "F.Cu") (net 11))
 (segment (start 69.465 71.255) (end 70.52 70.2) (width 0.2) (layer "F.Cu") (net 11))
 (segment (start 77.62 65.8) (end 82.02 70.2) (width 0.2) (layer "F.Cu") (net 11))
 (segment (start 76.94 70.2) (end 77.995 71.255) (width 0.2) (layer "F.Cu") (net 11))
 (segment (start 54 70.2) (end 55.055 71.255) (width 0.2) (layer "F.Cu") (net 11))
 (segment (start 74.42 65.8) (end 77.62 65.8) (width 0.2) (layer "F.Cu") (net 11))
 (segment (start 59.08 70.2) (end 60.135 71.255) (width 0.2) (layer "F.Cu") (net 11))
 (segment (start 77.995 71.255) (end 80.965 71.255) (width 0.2) (layer "F.Cu") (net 11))
 (segment (start 71.575 71.255) (end 75.885 71.255) (width 0.2) (layer "F.Cu") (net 11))
 (segment (start 70.52 69.98) (end 70.7 69.8) (width 0.2) (layer "F.Cu") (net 11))
 (segment (start 60.135 71.255) (end 64.385 71.255) (width 0.2) (layer "F.Cu") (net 11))
 (segment (start 66.495 71.255) (end 69.465 71.255) (width 0.2) (layer "F.Cu") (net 11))
 (segment (start 58.025 71.255) (end 59.08 70.2) (width 0.2) (layer "F.Cu") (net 11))
 (segment (start 64.385 71.255) (end 65.44 70.2) (width 0.2) (layer "F.Cu") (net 11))
 (segment (start 80.965 71.255) (end 82.02 70.2) (width 0.2) (layer "F.Cu") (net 11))
 (segment (start 65.44 70.2) (end 66.495 71.255) (width 0.2) (layer "F.Cu") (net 11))
 (segment (start 69.34 93.9) (end 72.93 90.31) (width 0.2) (layer "F.Cu") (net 6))
 (segment (start 72.93 90.31) (end 74.4 90.31) (width 0.2) (layer "F.Cu") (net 6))
 (segment (start 59.18 93.9) (end 56.76 93.9) (width 0.2) (layer "F.Cu") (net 1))
 (segment (start 56.76 93.9) (end 53.17 90.31) (width 0.2) (layer "F.Cu") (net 1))
 (segment (start 53.17 90.31) (end 51.5 90.31) (width 0.2) (layer "F.Cu") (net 1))
 (segment (start 66.8 93.9) (end 68 92.7) (width 0.2) (layer "F.Cu") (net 5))
 (segment (start 68 92.7) (end 68 90.31) (width 0.2) (layer "F.Cu") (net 5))
 (segment (start 62.9 92.54) (end 62.9 90.3) (width 0.2) (layer "F.Cu") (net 4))
 (segment (start 64.26 93.9) (end 62.9 92.54) (width 0.2) (layer "F.Cu") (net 4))
 (segment (start 61.72 93.9) (end 58.13 90.31) (width 0.2) (layer "F.Cu") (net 3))
 (segment (start 58.13 90.31) (end 56.6 90.31) (width 0.2) (layer "F.Cu") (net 3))
 (segment (start 66.495 79.305) (end 69.465 79.305) (width 0.2) (layer "F.Cu") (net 8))
 (segment (start 78.4 93.9) (end 82.02 90.28) (width 0.2) (layer "F.Cu") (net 8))
 (segment (start 69.465 79.305) (end 70.52 80.36) (width 0.2) (layer "F.Cu") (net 8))
 (segment (start 54 80.36) (end 55.055 79.305) (width 0.2) (layer "F.Cu") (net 8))
 (segment (start 71.575 79.305) (end 75.885 79.305) (width 0.2) (layer "F.Cu") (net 8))
 (segment (start 80.965 79.305) (end 82.02 80.36) (width 0.2) (layer "F.Cu") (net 8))
 (segment (start 75.885 79.305) (end 76.94 80.36) (width 0.2) (layer "F.Cu") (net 8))
 (segment (start 55.055 79.305) (end 58.025 79.305) (width 0.2) (layer "F.Cu") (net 8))
 (segment (start 64.385 79.305) (end 65.44 80.36) (width 0.2) (layer "F.Cu") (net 8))
 (segment (start 82.02 90.28) (end 82.02 80.36) (width 0.2) (layer "F.Cu") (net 8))
 (segment (start 76.94 80.36) (end 77.995 79.305) (width 0.2) (layer "F.Cu") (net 8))
 (segment (start 70.52 80.36) (end 71.575 79.305) (width 0.2) (layer "F.Cu") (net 8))
 (segment (start 77.995 79.305) (end 80.965 79.305) (width 0.2) (layer "F.Cu") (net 8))
 (segment (start 65.44 80.36) (end 66.495 79.305) (width 0.2) (layer "F.Cu") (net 8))
 (segment (start 59.08 80.36) (end 60.135 79.305) (width 0.2) (layer "F.Cu") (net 8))
 (segment (start 74.42 93.9) (end 78.4 93.9) (width 0.2) (layer "F.Cu") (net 8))
 (segment (start 60.135 79.305) (end 64.385 79.305) (width 0.2) (layer "F.Cu") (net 8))
 (segment (start 58.025 79.305) (end 59.08 80.36) (width 0.2) (layer "F.Cu") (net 8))
 (segment (start 73.78 92) (end 77.81 92) (width 0.2) (layer "F.Cu") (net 7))
 (segment (start 71.88 93.9) (end 73.78 92) (width 0.2) (layer "F.Cu") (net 7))
 (segment (start 77.81 92) (end 79.5 90.31) (width 0.2) (layer "F.Cu") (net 7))
 (segment (start 51.46 82.65) (end 51.5 82.69) (width 0.2) (layer "F.Cu") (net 2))
 (segment (start 51.46 80.36) (end 51.46 82.65) (width 0.2) (layer "F.Cu") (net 2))
 (segment (start 56.54 82.63) (end 56.6 82.69) (width 0.2) (layer "F.Cu") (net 18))
 (segment (start 56.54 80.36) (end 56.54 82.63) (width 0.2) (layer "F.Cu") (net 18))
 (segment (start 67.98 82.67) (end 68 82.69) (width 0.2) (layer "F.Cu") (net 20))
 (segment (start 67.98 80.36) (end 67.98 82.67) (width 0.2) (layer "F.Cu") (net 20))
 (segment (start 62.9 80.36) (end 62.9 82.68) (width 0.2) (layer "F.Cu") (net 19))
 (segment (start 79.48 80.36) (end 79.48 82.67) (width 0.2) (layer "F.Cu") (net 10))
 (segment (start 79.48 82.67) (end 79.5 82.69) (width 0.2) (layer "F.Cu") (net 10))
 (segment (start 74.4 80.36) (end 74.4 82.69) (width 0.2) (layer "F.Cu") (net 9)))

